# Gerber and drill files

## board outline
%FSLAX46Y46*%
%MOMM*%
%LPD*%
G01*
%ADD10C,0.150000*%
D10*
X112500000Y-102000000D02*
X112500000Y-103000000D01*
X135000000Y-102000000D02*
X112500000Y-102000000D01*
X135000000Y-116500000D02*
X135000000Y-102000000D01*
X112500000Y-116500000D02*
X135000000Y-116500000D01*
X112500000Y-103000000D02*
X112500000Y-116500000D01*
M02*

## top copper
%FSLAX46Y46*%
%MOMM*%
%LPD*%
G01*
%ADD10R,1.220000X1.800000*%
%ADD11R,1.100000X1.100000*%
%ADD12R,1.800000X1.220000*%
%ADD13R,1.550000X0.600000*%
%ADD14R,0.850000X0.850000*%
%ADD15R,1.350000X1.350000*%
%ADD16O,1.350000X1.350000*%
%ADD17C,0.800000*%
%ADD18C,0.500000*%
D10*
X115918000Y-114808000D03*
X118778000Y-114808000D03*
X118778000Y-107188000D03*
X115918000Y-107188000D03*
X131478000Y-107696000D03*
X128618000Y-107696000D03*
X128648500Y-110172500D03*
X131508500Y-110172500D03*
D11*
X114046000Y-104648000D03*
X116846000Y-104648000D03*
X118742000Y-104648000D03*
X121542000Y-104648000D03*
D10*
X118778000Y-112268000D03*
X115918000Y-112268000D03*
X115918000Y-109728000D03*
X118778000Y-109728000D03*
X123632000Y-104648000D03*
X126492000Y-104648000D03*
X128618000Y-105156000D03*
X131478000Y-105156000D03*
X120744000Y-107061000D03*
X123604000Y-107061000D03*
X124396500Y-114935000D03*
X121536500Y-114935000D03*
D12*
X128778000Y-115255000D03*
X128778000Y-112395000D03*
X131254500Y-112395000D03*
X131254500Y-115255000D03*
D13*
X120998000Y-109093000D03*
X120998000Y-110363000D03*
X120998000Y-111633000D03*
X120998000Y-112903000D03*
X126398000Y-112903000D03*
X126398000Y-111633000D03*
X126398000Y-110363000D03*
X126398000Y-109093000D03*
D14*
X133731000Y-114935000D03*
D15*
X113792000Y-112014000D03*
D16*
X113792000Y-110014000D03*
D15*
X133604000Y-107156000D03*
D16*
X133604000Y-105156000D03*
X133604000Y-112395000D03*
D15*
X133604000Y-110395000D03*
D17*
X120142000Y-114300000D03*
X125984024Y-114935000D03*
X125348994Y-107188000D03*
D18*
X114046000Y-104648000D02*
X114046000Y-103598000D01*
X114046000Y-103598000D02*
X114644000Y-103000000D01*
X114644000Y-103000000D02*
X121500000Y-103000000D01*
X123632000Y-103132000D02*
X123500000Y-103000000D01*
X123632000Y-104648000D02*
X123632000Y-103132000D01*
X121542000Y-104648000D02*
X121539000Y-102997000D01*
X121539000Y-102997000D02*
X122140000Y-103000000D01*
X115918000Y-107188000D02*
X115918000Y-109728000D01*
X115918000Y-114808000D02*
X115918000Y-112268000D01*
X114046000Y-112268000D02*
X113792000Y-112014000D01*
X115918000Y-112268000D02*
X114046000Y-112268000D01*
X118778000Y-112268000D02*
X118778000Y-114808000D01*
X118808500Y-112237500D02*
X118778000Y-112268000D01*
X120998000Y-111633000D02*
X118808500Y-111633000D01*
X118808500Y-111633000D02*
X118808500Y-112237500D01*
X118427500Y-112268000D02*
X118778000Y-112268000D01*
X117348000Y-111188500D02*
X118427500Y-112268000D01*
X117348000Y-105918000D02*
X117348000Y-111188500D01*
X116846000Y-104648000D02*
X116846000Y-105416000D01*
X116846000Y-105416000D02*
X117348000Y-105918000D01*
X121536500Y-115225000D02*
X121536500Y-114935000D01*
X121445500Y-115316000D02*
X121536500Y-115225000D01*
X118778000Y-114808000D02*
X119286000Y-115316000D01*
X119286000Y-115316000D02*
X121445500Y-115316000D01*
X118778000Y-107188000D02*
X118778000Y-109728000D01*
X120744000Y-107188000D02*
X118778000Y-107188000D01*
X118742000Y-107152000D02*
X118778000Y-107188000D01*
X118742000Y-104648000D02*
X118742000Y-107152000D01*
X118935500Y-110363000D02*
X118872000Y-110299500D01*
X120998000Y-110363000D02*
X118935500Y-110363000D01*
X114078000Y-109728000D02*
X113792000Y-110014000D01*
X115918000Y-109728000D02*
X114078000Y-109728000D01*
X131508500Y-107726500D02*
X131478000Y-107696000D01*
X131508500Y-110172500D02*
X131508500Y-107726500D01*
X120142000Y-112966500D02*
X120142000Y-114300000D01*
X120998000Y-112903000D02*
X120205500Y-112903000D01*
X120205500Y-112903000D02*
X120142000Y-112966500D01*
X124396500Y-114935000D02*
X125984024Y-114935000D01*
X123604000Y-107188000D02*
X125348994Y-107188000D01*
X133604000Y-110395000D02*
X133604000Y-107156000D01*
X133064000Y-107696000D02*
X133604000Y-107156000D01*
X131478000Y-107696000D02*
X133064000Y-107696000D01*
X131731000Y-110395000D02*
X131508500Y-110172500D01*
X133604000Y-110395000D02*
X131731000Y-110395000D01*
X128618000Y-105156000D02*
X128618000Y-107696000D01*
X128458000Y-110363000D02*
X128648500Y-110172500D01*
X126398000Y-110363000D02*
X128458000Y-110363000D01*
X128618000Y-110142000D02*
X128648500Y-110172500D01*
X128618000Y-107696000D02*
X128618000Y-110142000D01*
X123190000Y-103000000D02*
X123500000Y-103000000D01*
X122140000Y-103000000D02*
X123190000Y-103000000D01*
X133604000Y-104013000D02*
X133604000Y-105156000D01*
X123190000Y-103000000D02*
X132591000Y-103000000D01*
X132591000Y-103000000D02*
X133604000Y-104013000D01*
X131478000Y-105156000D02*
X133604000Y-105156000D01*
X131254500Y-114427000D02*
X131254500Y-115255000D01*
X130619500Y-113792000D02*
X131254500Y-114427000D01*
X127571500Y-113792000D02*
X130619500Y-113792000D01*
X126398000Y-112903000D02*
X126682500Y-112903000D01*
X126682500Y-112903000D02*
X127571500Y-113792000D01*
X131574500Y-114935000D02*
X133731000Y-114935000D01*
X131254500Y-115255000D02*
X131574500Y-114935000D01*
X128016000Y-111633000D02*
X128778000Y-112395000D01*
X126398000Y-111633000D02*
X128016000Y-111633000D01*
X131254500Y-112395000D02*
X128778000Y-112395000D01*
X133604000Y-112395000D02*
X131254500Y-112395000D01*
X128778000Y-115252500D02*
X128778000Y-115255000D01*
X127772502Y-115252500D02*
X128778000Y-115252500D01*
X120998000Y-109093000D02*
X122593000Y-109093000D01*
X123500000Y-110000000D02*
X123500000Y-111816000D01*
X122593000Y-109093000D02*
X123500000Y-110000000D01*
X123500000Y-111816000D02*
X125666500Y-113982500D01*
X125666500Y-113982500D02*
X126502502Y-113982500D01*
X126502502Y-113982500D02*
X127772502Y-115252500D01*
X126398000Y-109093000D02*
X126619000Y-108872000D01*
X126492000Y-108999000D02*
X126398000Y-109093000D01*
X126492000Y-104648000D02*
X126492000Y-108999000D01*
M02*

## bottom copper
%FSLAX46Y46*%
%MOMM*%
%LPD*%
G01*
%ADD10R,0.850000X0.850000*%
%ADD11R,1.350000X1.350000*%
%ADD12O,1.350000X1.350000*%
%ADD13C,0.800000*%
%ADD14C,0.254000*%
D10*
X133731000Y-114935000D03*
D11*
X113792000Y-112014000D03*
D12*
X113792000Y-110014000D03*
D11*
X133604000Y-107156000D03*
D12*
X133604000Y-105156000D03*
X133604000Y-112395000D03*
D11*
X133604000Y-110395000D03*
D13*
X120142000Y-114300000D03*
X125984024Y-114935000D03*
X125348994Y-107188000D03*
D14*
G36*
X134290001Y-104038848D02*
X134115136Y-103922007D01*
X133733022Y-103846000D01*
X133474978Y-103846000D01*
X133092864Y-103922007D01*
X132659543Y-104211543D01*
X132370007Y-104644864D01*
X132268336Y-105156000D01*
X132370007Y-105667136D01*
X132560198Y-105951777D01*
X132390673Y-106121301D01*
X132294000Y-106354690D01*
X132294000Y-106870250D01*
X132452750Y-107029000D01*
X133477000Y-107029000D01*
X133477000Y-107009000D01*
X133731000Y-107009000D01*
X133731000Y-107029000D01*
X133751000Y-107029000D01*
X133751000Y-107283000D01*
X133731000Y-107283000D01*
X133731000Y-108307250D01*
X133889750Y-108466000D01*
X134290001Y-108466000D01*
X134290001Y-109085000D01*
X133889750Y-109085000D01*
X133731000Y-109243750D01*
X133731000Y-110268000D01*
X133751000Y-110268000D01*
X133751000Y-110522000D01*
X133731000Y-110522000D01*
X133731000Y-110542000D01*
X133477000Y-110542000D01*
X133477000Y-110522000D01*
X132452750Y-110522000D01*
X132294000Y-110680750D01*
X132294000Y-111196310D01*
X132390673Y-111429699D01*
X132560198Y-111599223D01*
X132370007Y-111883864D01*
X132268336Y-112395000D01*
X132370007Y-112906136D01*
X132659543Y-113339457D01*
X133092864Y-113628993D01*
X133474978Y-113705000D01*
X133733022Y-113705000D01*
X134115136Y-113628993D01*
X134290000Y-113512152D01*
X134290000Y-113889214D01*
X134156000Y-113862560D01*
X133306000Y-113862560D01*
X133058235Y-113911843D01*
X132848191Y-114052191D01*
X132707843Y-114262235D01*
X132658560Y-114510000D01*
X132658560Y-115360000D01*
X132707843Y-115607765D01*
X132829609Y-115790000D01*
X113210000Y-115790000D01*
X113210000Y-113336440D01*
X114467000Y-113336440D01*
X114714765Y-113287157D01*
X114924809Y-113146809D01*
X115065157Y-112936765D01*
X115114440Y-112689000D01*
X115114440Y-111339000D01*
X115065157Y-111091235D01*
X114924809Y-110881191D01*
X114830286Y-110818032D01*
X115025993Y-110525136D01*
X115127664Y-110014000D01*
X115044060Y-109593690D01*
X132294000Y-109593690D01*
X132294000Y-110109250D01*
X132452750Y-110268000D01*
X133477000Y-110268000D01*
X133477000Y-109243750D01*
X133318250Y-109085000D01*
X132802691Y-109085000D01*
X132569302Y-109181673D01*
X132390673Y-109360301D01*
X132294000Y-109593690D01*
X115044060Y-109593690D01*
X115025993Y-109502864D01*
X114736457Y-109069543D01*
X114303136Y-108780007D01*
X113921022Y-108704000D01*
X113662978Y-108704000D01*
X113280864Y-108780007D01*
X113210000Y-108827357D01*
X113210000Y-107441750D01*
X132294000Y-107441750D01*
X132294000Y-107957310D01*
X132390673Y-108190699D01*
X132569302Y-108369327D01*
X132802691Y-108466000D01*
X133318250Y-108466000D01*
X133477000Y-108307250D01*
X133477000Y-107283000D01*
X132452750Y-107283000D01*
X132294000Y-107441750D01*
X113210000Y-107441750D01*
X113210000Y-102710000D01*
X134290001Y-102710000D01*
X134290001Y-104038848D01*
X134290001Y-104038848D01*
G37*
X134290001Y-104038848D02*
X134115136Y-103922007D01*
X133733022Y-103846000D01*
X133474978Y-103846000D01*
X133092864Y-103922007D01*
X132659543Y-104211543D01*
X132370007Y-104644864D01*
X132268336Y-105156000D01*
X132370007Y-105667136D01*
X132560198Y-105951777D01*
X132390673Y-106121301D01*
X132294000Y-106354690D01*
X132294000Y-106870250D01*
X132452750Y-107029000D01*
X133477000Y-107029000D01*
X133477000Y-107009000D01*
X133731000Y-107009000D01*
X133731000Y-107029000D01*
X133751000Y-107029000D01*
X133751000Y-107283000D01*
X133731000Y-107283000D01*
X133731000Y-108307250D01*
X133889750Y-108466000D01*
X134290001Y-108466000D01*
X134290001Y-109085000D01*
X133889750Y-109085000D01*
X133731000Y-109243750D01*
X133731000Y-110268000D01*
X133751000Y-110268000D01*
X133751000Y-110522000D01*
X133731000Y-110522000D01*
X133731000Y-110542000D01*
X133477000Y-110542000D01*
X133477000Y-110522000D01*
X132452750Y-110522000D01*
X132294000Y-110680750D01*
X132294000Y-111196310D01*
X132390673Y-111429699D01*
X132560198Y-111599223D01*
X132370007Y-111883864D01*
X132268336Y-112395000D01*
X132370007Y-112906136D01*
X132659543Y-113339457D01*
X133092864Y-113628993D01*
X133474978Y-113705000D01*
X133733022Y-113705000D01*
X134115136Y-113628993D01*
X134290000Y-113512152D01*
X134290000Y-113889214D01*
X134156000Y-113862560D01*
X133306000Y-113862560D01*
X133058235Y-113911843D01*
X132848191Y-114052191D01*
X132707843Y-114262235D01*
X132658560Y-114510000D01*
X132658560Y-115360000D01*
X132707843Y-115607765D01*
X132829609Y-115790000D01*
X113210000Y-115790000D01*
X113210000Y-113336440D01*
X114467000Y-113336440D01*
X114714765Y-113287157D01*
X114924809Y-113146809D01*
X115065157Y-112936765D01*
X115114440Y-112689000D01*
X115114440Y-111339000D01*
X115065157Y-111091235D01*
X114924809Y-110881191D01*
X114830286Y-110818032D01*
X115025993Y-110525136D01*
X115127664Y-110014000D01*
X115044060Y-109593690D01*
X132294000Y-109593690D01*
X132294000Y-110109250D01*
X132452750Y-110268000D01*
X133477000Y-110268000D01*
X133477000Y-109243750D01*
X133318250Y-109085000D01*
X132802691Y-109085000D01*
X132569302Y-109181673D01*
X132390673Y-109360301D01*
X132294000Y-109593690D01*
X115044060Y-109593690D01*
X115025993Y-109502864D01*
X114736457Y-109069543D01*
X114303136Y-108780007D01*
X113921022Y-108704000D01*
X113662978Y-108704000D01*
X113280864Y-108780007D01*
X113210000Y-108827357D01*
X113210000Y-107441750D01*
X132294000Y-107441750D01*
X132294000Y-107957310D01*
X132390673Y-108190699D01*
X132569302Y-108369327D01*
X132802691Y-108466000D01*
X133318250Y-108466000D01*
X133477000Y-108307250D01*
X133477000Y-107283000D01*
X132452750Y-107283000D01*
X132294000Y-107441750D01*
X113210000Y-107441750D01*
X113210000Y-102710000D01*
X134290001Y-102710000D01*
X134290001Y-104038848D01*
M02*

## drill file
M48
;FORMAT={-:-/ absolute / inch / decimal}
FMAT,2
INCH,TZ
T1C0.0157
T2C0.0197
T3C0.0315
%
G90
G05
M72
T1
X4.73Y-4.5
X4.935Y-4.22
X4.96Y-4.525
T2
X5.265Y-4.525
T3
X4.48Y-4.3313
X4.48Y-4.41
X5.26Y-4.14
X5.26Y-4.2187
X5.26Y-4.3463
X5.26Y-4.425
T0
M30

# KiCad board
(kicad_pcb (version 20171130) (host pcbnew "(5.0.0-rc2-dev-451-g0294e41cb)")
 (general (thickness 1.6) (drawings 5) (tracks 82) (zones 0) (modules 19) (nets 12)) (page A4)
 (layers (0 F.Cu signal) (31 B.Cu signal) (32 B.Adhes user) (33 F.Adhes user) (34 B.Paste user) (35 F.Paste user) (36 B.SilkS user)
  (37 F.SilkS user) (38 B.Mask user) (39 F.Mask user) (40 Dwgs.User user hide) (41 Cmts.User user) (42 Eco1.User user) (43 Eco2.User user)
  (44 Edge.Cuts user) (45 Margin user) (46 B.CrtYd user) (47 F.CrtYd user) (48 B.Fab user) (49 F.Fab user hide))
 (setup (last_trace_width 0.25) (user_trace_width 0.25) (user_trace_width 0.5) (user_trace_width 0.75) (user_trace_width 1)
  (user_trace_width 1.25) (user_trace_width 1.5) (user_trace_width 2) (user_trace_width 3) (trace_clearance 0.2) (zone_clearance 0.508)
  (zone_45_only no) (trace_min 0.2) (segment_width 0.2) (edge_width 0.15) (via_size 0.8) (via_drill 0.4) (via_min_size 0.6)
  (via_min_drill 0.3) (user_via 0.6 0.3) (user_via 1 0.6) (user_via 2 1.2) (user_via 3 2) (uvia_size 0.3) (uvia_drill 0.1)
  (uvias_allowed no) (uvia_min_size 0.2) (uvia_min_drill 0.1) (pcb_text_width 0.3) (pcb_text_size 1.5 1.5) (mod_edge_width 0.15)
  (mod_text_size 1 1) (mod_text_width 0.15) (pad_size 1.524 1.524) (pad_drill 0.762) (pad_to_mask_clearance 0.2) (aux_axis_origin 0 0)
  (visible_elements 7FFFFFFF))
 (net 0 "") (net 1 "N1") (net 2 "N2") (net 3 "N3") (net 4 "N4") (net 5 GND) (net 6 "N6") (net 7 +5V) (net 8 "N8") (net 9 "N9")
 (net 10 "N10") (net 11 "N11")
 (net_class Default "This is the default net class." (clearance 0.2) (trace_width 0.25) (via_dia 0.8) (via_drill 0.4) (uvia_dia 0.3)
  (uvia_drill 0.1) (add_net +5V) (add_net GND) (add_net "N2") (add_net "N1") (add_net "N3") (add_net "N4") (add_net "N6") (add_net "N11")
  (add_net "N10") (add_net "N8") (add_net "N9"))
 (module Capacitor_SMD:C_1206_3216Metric (layer F.Cu) (at 117.348 114.808 180)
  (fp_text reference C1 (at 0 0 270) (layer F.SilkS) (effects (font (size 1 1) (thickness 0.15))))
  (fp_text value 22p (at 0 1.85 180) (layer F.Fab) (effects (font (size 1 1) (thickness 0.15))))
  (pad 2 smd rect (at 1.43 0 180) (size 1.22 1.8) (layers F.Cu F.Paste F.Mask) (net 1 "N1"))
  (pad 1 smd rect (at -1.43 0 180) (size 1.22 1.8) (layers F.Cu F.Paste F.Mask) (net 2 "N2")))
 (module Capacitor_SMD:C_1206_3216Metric (layer F.Cu) (at 117.348 107.188 180)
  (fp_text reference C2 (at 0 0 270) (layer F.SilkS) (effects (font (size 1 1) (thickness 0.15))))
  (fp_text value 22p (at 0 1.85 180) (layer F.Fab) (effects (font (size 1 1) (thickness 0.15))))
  (pad 1 smd rect (at -1.43 0 180) (size 1.22 1.8) (layers F.Cu F.Paste F.Mask) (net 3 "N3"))
  (pad 2 smd rect (at 1.43 0 180) (size 1.22 1.8) (layers F.Cu F.Paste F.Mask) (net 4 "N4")))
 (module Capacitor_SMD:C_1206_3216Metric (layer F.Cu) (at 130.048 107.696)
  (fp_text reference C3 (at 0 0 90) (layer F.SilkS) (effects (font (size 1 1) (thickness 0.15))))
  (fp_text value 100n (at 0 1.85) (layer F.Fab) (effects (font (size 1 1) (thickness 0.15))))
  (pad 2 smd rect (at 1.43 0) (size 1.22 1.8) (layers F.Cu F.Paste F.Mask) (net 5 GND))
  (pad 1 smd rect (at -1.43 0) (size 1.22 1.8) (layers F.Cu F.Paste F.Mask) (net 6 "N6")))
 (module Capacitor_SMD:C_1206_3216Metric (layer F.Cu) (at 130.0785 110.1725)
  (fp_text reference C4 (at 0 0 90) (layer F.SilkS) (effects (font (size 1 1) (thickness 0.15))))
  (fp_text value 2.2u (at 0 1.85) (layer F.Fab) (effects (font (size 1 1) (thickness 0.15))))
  (pad 1 smd rect (at -1.43 0) (size 1.22 1.8) (layers F.Cu F.Paste F.Mask) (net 6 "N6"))
  (pad 2 smd rect (at 1.43 0) (size 1.22 1.8) (layers F.Cu F.Paste F.Mask) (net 5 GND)))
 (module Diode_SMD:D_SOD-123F (layer F.Cu) (at 115.446 104.648)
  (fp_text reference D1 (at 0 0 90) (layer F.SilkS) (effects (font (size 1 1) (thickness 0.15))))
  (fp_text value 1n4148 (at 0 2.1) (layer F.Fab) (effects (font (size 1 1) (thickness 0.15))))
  (pad 1 smd rect (at -1.4 0) (size 1.1 1.1) (layers F.Cu F.Paste F.Mask) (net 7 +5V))
  (pad 2 smd rect (at 1.4 0) (size 1.1 1.1) (layers F.Cu F.Paste F.Mask) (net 2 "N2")))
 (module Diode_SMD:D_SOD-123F (layer F.Cu) (at 120.142 104.648 180)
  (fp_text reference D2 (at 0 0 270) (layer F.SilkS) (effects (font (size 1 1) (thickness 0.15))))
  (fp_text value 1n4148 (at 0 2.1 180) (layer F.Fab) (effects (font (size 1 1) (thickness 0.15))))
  (pad 2 smd rect (at 1.4 0 180) (size 1.1 1.1) (layers F.Cu F.Paste F.Mask) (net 3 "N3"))
  (pad 1 smd rect (at -1.4 0 180) (size 1.1 1.1) (layers F.Cu F.Paste F.Mask) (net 7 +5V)))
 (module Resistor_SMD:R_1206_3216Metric (layer F.Cu) (at 117.348 112.268 180)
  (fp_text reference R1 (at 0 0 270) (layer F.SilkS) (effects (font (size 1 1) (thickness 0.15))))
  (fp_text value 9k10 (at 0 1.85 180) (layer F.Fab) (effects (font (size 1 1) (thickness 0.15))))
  (pad 1 smd rect (at -1.43 0 180) (size 1.22 1.8) (layers F.Cu F.Paste F.Mask) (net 2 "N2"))
  (pad 2 smd rect (at 1.43 0 180) (size 1.22 1.8) (layers F.Cu F.Paste F.Mask) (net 1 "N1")))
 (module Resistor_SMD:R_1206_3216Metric (layer F.Cu) (at 117.348 109.728 180)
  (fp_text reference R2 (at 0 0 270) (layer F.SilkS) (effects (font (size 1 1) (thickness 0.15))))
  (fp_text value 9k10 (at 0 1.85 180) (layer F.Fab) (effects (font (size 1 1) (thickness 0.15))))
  (pad 2 smd rect (at 1.43 0 180) (size 1.22 1.8) (layers F.Cu F.Paste F.Mask) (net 4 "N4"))
  (pad 1 smd rect (at -1.43 0 180) (size 1.22 1.8) (layers F.Cu F.Paste F.Mask) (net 3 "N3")))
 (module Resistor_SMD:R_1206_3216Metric (layer F.Cu) (at 125.062 104.648 180)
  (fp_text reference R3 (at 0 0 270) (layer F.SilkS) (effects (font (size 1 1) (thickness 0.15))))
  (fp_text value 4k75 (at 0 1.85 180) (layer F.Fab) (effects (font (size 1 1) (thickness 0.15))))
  (pad 2 smd rect (at 1.43 0 180) (size 1.22 1.8) (layers F.Cu F.Paste F.Mask) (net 7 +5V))
  (pad 1 smd rect (at -1.43 0 180) (size 1.22 1.8) (layers F.Cu F.Paste F.Mask) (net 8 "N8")))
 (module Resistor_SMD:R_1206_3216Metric (layer F.Cu) (at 130.048 105.156)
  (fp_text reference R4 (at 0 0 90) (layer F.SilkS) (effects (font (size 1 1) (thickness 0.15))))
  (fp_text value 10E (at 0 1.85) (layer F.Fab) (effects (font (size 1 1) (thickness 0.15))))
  (pad 1 smd rect (at -1.43 0) (size 1.22 1.8) (layers F.Cu F.Paste F.Mask) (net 6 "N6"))
  (pad 2 smd rect (at 1.43 0) (size 1.22 1.8) (layers F.Cu F.Paste F.Mask) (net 7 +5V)))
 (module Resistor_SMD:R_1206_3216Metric (layer F.Cu) (at 122.174 107.061 180)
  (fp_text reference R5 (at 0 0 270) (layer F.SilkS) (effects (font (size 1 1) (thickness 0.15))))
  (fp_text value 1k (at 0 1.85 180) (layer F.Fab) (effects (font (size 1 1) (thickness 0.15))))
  (pad 2 smd rect (at 1.43 0 180) (size 1.22 1.8) (layers F.Cu F.Paste F.Mask) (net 3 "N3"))
  (pad 1 smd rect (at -1.43 0 180) (size 1.22 1.8) (layers F.Cu F.Paste F.Mask) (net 5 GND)))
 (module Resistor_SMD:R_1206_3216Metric (layer F.Cu) (at 122.9665 114.935 180)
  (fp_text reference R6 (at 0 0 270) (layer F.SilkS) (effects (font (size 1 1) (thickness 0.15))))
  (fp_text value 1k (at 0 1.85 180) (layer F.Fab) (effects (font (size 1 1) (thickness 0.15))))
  (pad 1 smd rect (at -1.43 0 180) (size 1.22 1.8) (layers F.Cu F.Paste F.Mask) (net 5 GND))
  (pad 2 smd rect (at 1.43 0 180) (size 1.22 1.8) (layers F.Cu F.Paste F.Mask) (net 2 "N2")))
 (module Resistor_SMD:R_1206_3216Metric (layer F.Cu) (at 128.778 113.825 90)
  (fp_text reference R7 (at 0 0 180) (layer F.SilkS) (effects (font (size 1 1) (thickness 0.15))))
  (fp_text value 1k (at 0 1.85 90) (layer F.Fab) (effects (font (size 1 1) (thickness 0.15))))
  (pad 1 smd rect (at -1.43 0 90) (size 1.22 1.8) (layers F.Cu F.Paste F.Mask) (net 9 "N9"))
  (pad 2 smd rect (at 1.43 0 90) (size 1.22 1.8) (layers F.Cu F.Paste F.Mask) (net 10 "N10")))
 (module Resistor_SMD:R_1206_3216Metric (layer F.Cu) (at 131.2545 113.825 90)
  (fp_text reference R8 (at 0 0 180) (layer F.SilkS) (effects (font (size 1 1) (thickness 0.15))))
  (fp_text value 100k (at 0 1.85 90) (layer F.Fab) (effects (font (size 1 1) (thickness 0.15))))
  (pad 2 smd rect (at 1.43 0 90) (size 1.22 1.8) (layers F.Cu F.Paste F.Mask) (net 9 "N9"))
  (pad 1 smd rect (at -1.43 0 90) (size 1.22 1.8) (layers F.Cu F.Paste F.Mask) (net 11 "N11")))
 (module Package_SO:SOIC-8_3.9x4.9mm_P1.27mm (layer F.Cu) (at 123.698 110.998)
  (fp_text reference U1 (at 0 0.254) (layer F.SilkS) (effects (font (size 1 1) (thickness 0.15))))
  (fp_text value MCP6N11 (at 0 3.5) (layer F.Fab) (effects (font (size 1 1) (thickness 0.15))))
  (pad 1 smd rect (at -2.7 -1.905) (size 1.55 0.6) (layers F.Cu F.Paste F.Mask) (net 9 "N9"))
  (pad 2 smd rect (at -2.7 -0.635) (size 1.55 0.6) (layers F.Cu F.Paste F.Mask) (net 3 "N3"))
  (pad 3 smd rect (at -2.7 0.635) (size 1.55 0.6) (layers F.Cu F.Paste F.Mask) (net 2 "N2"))
  (pad 4 smd rect (at -2.7 1.905) (size 1.55 0.6) (layers F.Cu F.Paste F.Mask) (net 5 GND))
  (pad 5 smd rect (at 2.7 1.905) (size 1.55 0.6) (layers F.Cu F.Paste F.Mask) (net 11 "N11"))
  (pad 6 smd rect (at 2.7 0.635) (size 1.55 0.6) (layers F.Cu F.Paste F.Mask) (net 10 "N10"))
  (pad 7 smd rect (at 2.7 -0.635) (size 1.55 0.6) (layers F.Cu F.Paste F.Mask) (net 6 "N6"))
  (pad 8 smd rect (at 2.7 -1.905) (size 1.55 0.6) (layers F.Cu F.Paste F.Mask) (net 8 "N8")))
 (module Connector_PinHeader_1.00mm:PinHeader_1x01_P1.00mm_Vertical (layer F.Cu) (at 133.731 114.935 270)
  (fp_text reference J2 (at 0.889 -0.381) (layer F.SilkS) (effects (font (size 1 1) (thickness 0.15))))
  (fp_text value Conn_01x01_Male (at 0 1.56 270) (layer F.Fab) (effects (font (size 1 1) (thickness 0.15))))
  (pad 1 thru_hole rect (at 0 0 270) (size 0.85 0.85) (drill 0.5) (layers *.Cu *.Mask) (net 11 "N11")))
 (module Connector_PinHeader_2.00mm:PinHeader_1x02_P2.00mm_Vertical (layer F.Cu) (at 113.792 112.014 180)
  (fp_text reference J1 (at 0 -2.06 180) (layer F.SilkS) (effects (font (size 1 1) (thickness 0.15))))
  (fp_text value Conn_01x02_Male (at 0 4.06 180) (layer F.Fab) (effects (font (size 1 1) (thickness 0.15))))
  (pad 1 thru_hole rect (at 0 0 180) (size 1.35 1.35) (drill 0.8) (layers *.Cu *.Mask) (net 1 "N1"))
  (pad 2 thru_hole oval (at 0 2 180) (size 1.35 1.35) (drill 0.8) (layers *.Cu *.Mask) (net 4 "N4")))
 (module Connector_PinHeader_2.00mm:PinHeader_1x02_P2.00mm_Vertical (layer F.Cu) (at 133.604 107.156 180)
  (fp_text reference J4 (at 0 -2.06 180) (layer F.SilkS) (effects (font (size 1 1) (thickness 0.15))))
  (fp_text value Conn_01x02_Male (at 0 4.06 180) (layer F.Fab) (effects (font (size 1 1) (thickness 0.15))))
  (pad 1 thru_hole rect (at 0 0 180) (size 1.35 1.35) (drill 0.8) (layers *.Cu *.Mask) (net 5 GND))
  (pad 2 thru_hole oval (at 0 2 180) (size 1.35 1.35) (drill 0.8) (layers *.Cu *.Mask) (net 7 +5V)))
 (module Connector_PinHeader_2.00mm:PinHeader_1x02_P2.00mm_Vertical (layer F.Cu) (at 133.604 110.395)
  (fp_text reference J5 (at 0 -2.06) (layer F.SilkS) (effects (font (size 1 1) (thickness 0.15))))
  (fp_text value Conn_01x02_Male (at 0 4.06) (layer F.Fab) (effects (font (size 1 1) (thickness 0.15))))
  (pad 2 thru_hole oval (at 0 2) (size 1.35 1.35) (drill 0.8) (layers *.Cu *.Mask) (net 10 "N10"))
  (pad 1 thru_hole rect (at 0 0) (size 1.35 1.35) (drill 0.8) (layers *.Cu *.Mask) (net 5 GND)))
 (gr_line (start 112.5 102) (end 112.5 103) (layer Edge.Cuts) (width 0.15))
 (gr_line (start 135 102) (end 112.5 102) (layer Edge.Cuts) (width 0.15))
 (gr_line (start 135 116.5) (end 135 102) (layer Edge.Cuts) (width 0.15))
 (gr_line (start 112.5 116.5) (end 135 116.5) (layer Edge.Cuts) (width 0.15))
 (gr_line (start 112.5 103) (end 112.5 116.5) (layer Edge.Cuts) (width 0.15))
 (segment (start 114.046 104.648) (end 114.046 103.598) (width 0.5) (layer F.Cu) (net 7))
 (segment (start 114.046 103.598) (end 114.644 103) (width 0.5) (layer F.Cu) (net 7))
 (segment (start 114.644 103) (end 121.5 103) (width 0.5) (layer F.Cu) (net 7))
 (segment (start 123.632 103.132) (end 123.5 103) (width 0.5) (layer F.Cu) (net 7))
 (segment (start 123.632 104.648) (end 123.632 103.132) (width 0.5) (layer F.Cu) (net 7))
 (segment (start 121.542 104.648) (end 121.539 102.997) (width 0.5) (layer F.Cu) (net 7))
 (segment (start 121.539 102.997) (end 122.14 103) (width 0.5) (layer F.Cu) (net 7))
 (segment (start 115.918 107.188) (end 115.918 109.728) (width 0.5) (layer F.Cu) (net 4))
 (segment (start 115.918 114.808) (end 115.918 112.268) (width 0.5) (layer F.Cu) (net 1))
 (segment (start 114.046 112.268) (end 113.792 112.014) (width 0.5) (layer F.Cu) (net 1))
 (segment (start 115.918 112.268) (end 114.046 112.268) (width 0.5) (layer F.Cu) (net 1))
 (segment (start 118.778 112.268) (end 118.778 114.808) (width 0.5) (layer F.Cu) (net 2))
 (segment (start 118.8085 112.2375) (end 118.778 112.268) (width 0.5) (layer F.Cu) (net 2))
 (segment (start 120.998 111.633) (end 118.8085 111.633) (width 0.5) (layer F.Cu) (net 2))
 (segment (start 118.8085 111.633) (end 118.8085 112.2375) (width 0.5) (layer F.Cu) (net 2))
 (segment (start 118.4275 112.268) (end 118.778 112.268) (width 0.5) (layer F.Cu) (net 2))
 (segment (start 117.348 111.1885) (end 118.4275 112.268) (width 0.5) (layer F.Cu) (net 2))
 (segment (start 117.348 105.918) (end 117.348 111.1885) (width 0.5) (layer F.Cu) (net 2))
 (segment (start 116.846 104.648) (end 116.846 105.416) (width 0.5) (layer F.Cu) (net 2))
 (segment (start 116.846 105.416) (end 117.348 105.918) (width 0.5) (layer F.Cu) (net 2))
 (segment (start 121.5365 115.225) (end 121.5365 114.935) (width 0.5) (layer F.Cu) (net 2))
 (segment (start 121.4455 115.316) (end 121.5365 115.225) (width 0.5) (layer F.Cu) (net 2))
 (segment (start 118.778 114.808) (end 119.286 115.316) (width 0.5) (layer F.Cu) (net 2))
 (segment (start 119.286 115.316) (end 121.4455 115.316) (width 0.5) (layer F.Cu) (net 2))
 (segment (start 118.778 107.188) (end 118.778 109.728) (width 0.5) (layer F.Cu) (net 3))
 (segment (start 120.744 107.188) (end 118.778 107.188) (width 0.5) (layer F.Cu) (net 3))
 (segment (start 118.742 107.152) (end 118.778 107.188) (width 0.5) (layer F.Cu) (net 3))
 (segment (start 118.742 104.648) (end 118.742 107.152) (width 0.5) (layer F.Cu) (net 3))
 (segment (start 118.9355 110.363) (end 118.872 110.2995) (width 0.5) (layer F.Cu) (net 3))
 (segment (start 120.998 110.363) (end 118.9355 110.363) (width 0.5) (layer F.Cu) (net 3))
 (segment (start 114.078 109.728) (end 113.792 110.014) (width 0.5) (layer F.Cu) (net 4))
 (segment (start 115.918 109.728) (end 114.078 109.728) (width 0.5) (layer F.Cu) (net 4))
 (segment (start 131.5085 107.7265) (end 131.478 107.696) (width 0.5) (layer F.Cu) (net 5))
 (segment (start 131.5085 110.1725) (end 131.5085 107.7265) (width 0.5) (layer F.Cu) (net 5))
 (via (at 120.142 114.3) (size 0.8) (drill 0.4) (layers F.Cu B.Cu) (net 5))
 (segment (start 120.142 112.9665) (end 120.142 114.3) (width 0.5) (layer F.Cu) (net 5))
 (segment (start 120.998 112.903) (end 120.2055 112.903) (width 0.5) (layer F.Cu) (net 5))
 (segment (start 120.2055 112.903) (end 120.142 112.9665) (width 0.5) (layer F.Cu) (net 5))
 (via (at 125.984024 114.935) (size 0.8) (drill 0.4) (layers F.Cu B.Cu) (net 5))
 (segment (start 124.3965 114.935) (end 125.984024 114.935) (width 0.5) (layer F.Cu) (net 5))
 (via (at 125.348994 107.188) (size 0.8) (drill 0.4) (layers F.Cu B.Cu) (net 5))
 (segment (start 123.604 107.188) (end 125.348994 107.188) (width 0.5) (layer F.Cu) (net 5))
 (segment (start 133.604 110.395) (end 133.604 107.156) (width 0.5) (layer F.Cu) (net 5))
 (segment (start 133.064 107.696) (end 133.604 107.156) (width 0.5) (layer F.Cu) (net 5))
 (segment (start 131.478 107.696) (end 133.064 107.696) (width 0.5) (layer F.Cu) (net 5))
 (segment (start 131.731 110.395) (end 131.5085 110.1725) (width 0.5) (layer F.Cu) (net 5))
 (segment (start 133.604 110.395) (end 131.731 110.395) (width 0.5) (layer F.Cu) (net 5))
 (segment (start 128.618 105.156) (end 128.618 107.696) (width 0.5) (layer F.Cu) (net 6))
 (segment (start 128.458 110.363) (end 128.6485 110.1725) (width 0.5) (layer F.Cu) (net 6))
 (segment (start 126.398 110.363) (end 128.458 110.363) (width 0.5) (layer F.Cu) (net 6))
 (segment (start 128.618 110.142) (end 128.6485 110.1725) (width 0.5) (layer F.Cu) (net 6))
 (segment (start 128.618 107.696) (end 128.618 110.142) (width 0.5) (layer F.Cu) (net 6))
 (segment (start 123.19 103) (end 123.5 103) (width 0.5) (layer F.Cu) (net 7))
 (segment (start 122.14 103) (end 123.19 103) (width 0.5) (layer F.Cu) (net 7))
 (segment (start 133.604 104.013) (end 133.604 105.156) (width 0.5) (layer F.Cu) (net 7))
 (segment (start 123.19 103) (end 132.591 103) (width 0.5) (layer F.Cu) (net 7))
 (segment (start 132.591 103) (end 133.604 104.013) (width 0.5) (layer F.Cu) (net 7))
 (segment (start 131.478 105.156) (end 133.604 105.156) (width 0.5) (layer F.Cu) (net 7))
 (segment (start 131.5745 114.935) (end 133.731 114.935) (width 0.5) (layer F.Cu) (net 11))
 (segment (start 131.2545 115.255) (end 131.5745 114.935) (width 0.5) (layer F.Cu) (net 11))
 (segment (start 131.0792 115.255) (end 131.2545 115.255) (width 0.5) (layer F.Cu) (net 11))
 (segment (start 129.6162 113.792) (end 131.0792 115.255) (width 0.5) (layer F.Cu) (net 11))
 (segment (start 127.5715 113.792) (end 129.6162 113.792) (width 0.5) (layer F.Cu) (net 11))
 (segment (start 126.398 112.903) (end 126.6825 112.903) (width 0.5) (layer F.Cu) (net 11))
 (segment (start 126.6825 112.903) (end 127.5715 113.792) (width 0.5) (layer F.Cu) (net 11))
 (segment (start 126.398 111.633) (end 128.016 111.633) (width 0.5) (layer F.Cu) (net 10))
 (segment (start 128.016 111.633) (end 128.778 112.395) (width 0.5) (layer F.Cu) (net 10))
 (segment (start 129.068 112.395) (end 128.778 112.395) (width 0.25) (layer F.Cu) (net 10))
 (segment (start 130.084 113.411) (end 129.068 112.395) (width 0.25) (layer F.Cu) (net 10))
 (segment (start 132.588 113.411) (end 130.084 113.411) (width 0.25) (layer F.Cu) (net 10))
 (segment (start 133.604 112.395) (end 132.588 113.411) (width 0.25) (layer F.Cu) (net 10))
 (segment (start 125.6665 113.9825) (end 126.502502 113.9825) (width 0.5) (layer F.Cu) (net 9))
 (segment (start 127.772502 115.2525) (end 128.778 115.2525) (width 0.5) (layer F.Cu) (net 9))
 (segment (start 123.5 111.816) (end 125.6665 113.9825) (width 0.5) (layer F.Cu) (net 9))
 (segment (start 128.778 115.2525) (end 128.778 115.255) (width 0.5) (layer F.Cu) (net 9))
 (segment (start 123.5 110) (end 123.5 111.816) (width 0.5) (layer F.Cu) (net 9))
 (segment (start 126.502502 113.9825) (end 127.772502 115.2525) (width 0.5) (layer F.Cu) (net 9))
 (segment (start 120.998 109.093) (end 122.593 109.093) (width 0.5) (layer F.Cu) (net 9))
 (segment (start 122.593 109.093) (end 123.5 110) (width 0.5) (layer F.Cu) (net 9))
 (segment (start 126.398 109.093) (end 126.619 108.872) (width 0.5) (layer F.Cu) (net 8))
 (segment (start 126.492 108.999) (end 126.398 109.093) (width 0.5) (layer F.Cu) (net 8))
 (segment (start 126.492 104.648) (end 126.492 108.999) (width 0.5) (layer F.Cu) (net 8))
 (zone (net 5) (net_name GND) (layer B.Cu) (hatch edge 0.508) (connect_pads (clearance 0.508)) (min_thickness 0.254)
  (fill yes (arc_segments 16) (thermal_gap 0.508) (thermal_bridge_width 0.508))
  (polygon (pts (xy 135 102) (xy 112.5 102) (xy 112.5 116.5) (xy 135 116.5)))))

